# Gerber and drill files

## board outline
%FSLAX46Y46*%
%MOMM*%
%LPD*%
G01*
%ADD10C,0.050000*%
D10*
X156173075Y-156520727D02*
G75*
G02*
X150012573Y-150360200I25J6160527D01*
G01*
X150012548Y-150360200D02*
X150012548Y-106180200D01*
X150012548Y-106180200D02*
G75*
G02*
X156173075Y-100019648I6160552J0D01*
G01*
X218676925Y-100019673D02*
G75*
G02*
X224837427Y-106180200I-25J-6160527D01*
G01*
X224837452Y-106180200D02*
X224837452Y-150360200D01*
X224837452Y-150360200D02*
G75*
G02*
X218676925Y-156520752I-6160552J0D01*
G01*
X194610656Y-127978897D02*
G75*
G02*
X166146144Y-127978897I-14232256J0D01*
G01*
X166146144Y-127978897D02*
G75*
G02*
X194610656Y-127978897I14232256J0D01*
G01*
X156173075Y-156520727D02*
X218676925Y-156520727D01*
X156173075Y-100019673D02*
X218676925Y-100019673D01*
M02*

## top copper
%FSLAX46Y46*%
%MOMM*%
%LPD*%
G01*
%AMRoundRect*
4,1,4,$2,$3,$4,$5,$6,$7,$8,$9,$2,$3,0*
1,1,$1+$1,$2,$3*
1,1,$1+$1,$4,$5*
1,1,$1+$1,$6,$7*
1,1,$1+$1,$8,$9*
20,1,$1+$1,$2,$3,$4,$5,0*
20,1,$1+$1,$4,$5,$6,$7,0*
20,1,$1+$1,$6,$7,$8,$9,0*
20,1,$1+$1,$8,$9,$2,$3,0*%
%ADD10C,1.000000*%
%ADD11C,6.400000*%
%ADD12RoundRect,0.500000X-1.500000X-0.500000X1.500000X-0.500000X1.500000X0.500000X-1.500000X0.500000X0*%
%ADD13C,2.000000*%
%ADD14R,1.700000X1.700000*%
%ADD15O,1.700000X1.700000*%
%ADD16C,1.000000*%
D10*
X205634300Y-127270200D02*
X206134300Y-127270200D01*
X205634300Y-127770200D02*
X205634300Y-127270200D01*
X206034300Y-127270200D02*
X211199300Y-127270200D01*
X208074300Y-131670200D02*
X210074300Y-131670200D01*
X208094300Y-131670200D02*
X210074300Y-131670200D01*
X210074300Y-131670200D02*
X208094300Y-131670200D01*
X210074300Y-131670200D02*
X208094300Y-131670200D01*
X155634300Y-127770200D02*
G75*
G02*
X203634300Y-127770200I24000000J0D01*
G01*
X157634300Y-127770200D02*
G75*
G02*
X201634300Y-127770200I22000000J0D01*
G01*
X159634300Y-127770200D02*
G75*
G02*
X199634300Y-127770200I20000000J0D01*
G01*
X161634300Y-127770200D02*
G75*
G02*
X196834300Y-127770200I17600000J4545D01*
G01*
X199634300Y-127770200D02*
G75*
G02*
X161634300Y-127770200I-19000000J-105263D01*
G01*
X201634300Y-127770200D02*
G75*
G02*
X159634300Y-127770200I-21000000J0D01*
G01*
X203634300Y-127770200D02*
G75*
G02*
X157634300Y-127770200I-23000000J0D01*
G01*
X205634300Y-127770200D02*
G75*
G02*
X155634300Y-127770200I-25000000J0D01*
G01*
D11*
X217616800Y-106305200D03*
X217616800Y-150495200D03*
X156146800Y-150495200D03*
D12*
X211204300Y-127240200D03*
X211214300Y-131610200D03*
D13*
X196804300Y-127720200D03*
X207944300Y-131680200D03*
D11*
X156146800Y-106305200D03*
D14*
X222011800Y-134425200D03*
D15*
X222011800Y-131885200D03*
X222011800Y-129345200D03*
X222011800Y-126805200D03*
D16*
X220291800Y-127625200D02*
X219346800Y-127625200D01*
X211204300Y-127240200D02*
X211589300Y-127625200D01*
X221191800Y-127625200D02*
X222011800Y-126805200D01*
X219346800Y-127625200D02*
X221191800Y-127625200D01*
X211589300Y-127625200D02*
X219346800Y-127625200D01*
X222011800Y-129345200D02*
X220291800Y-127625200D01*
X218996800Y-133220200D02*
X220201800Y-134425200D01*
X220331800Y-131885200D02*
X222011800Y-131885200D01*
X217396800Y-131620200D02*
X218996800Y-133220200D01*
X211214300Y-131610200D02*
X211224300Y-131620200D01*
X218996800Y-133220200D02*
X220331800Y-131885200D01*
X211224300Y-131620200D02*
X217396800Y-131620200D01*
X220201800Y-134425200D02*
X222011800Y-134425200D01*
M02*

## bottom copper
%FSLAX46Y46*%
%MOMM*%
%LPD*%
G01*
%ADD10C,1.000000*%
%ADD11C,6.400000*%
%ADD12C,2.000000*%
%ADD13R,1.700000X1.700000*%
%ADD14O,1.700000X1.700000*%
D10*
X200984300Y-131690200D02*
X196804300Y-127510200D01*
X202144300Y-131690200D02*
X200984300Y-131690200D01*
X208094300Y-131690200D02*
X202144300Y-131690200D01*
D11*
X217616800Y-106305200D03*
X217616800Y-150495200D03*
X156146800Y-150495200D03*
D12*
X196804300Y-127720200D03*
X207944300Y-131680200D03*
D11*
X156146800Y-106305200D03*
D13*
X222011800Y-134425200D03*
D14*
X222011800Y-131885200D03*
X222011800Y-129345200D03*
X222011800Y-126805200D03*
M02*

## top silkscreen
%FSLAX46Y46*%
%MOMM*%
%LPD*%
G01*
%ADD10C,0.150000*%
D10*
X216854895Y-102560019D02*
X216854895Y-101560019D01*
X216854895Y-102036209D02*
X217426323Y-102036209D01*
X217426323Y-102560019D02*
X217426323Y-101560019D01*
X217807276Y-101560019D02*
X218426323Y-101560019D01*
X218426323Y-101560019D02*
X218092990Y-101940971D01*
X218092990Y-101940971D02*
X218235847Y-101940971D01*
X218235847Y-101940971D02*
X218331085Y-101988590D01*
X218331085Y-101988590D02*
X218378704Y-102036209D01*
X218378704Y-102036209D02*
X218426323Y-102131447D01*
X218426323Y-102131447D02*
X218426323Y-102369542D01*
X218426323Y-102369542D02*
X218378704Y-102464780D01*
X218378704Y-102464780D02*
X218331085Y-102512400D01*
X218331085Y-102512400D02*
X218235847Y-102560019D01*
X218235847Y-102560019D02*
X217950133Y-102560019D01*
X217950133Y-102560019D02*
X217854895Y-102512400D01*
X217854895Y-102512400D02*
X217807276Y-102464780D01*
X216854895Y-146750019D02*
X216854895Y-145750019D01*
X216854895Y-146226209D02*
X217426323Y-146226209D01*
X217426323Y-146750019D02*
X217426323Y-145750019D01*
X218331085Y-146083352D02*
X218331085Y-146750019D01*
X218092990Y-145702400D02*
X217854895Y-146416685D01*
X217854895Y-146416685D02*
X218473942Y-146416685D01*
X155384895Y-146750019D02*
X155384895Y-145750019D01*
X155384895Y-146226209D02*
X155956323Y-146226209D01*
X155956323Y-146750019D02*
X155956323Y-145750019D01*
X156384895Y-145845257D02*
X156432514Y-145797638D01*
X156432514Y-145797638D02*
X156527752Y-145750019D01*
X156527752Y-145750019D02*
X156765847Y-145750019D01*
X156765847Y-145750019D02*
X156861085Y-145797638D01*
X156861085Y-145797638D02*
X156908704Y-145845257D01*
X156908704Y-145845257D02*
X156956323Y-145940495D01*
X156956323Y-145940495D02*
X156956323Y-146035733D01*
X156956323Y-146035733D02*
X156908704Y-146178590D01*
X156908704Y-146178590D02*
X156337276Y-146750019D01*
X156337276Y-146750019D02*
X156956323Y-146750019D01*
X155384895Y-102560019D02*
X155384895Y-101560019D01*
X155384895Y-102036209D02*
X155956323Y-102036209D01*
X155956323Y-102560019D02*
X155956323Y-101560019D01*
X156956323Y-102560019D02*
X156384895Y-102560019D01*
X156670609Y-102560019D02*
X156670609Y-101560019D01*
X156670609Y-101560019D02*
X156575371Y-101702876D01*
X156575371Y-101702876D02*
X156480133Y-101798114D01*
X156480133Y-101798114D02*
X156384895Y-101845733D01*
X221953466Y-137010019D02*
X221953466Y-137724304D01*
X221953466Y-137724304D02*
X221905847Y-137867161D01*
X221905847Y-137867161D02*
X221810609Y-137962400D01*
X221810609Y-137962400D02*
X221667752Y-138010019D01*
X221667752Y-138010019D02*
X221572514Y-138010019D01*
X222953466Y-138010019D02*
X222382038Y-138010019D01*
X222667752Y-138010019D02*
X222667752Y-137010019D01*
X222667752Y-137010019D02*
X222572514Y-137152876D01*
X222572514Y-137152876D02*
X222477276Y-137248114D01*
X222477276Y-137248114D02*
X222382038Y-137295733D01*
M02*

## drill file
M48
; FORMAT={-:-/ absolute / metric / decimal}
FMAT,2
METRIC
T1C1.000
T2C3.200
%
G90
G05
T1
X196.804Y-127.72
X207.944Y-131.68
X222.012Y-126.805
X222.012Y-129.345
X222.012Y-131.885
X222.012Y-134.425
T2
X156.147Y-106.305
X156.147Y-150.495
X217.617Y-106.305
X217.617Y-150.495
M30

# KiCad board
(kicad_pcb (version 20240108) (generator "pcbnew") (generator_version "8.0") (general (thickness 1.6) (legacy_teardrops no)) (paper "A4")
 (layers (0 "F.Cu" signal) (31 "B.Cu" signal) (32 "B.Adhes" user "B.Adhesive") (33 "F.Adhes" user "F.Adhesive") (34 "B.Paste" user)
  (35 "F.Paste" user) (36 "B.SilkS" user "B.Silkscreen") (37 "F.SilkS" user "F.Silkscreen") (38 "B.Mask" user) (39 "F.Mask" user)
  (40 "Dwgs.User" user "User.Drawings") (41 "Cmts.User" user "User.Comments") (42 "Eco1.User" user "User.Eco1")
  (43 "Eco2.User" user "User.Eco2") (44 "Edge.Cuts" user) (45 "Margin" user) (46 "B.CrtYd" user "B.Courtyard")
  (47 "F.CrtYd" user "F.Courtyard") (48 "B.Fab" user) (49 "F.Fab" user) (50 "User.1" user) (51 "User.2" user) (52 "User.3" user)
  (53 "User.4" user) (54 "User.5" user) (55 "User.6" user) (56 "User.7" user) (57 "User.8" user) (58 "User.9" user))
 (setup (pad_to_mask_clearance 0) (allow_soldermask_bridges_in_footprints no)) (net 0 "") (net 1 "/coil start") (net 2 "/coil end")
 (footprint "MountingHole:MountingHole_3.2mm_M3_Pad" (layer "F.Cu") (at 217.6168 106.3052)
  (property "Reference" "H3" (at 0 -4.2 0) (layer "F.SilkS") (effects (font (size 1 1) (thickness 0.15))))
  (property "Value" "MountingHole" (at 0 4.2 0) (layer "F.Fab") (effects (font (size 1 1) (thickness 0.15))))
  (pad "1" thru_hole circle (at 0 0) (size 6.4 6.4) (drill 3.2) (layers "*.Cu" "*.Mask") (remove_unused_layers no)))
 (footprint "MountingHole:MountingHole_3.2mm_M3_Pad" (layer "F.Cu") (at 217.6168 150.4952)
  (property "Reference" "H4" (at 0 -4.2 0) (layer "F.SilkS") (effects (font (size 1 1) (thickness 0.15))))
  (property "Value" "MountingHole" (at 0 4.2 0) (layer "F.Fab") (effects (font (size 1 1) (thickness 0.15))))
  (pad "1" thru_hole circle (at 0 0) (size 6.4 6.4) (drill 3.2) (layers "*.Cu" "*.Mask") (remove_unused_layers no)))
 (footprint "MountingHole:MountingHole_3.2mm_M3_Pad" (layer "F.Cu") (at 156.1468 150.4952)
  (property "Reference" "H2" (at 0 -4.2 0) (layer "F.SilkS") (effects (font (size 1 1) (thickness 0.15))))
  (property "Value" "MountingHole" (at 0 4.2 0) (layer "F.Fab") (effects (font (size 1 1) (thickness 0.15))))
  (pad "1" thru_hole circle (at 0 0) (size 6.4 6.4) (drill 3.2) (layers "*.Cu" "*.Mask") (remove_unused_layers no)))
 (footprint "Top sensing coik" (layer "F.Cu") (at 179.6343 127.7702)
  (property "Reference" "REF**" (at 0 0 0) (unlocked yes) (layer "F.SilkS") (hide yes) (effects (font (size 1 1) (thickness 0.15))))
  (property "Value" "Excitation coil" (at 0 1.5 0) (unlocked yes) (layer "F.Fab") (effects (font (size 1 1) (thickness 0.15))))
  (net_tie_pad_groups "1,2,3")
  (fp_line (start 26 -0.5) (end 26.5 -0.5) (stroke (width 1) (type solid)) (layer "F.Cu"))
  (fp_line (start 26 0) (end 26 -0.5) (stroke (width 1) (type solid)) (layer "F.Cu"))
  (fp_line (start 26.4 -0.5) (end 31.565 -0.5) (stroke (width 1) (type default)) (layer "F.Cu"))
  (fp_line (start 28.44 3.9) (end 30.44 3.9) (stroke (width 1) (type default)) (layer "F.Cu"))
  (fp_line (start 28.46 3.9) (end 30.44 3.9) (stroke (width 1) (type default)) (layer "F.Cu"))
  (fp_line (start 30.44 3.9) (end 28.46 3.9) (stroke (width 1) (type default)) (layer "F.Cu"))
  (fp_line (start 30.44 3.9) (end 28.46 3.9) (stroke (width 1) (type default)) (layer "F.Cu"))
  (fp_arc (start -24 0) (mid 0 -24) (end 24 0) (stroke (width 1) (type solid)) (layer "F.Cu"))
  (fp_arc (start -22 0) (mid 0 -22) (end 22 0) (stroke (width 1) (type solid)) (layer "F.Cu"))
  (fp_arc (start -20 0) (mid 0 -20) (end 20 0) (stroke (width 1) (type solid)) (layer "F.Cu"))
  (fp_arc (start -18 0) (mid -0.4 -17.604546) (end 17.2 0) (stroke (width 1) (type solid)) (layer "F.Cu"))
  (fp_arc (start 20 0) (mid 1 19.105555) (end -18 0) (stroke (width 1) (type solid)) (layer "F.Cu"))
  (fp_arc (start 22 0) (mid 1 21) (end -20 0) (stroke (width 1) (type solid)) (layer "F.Cu"))
  (fp_arc (start 24 0) (mid 1 23) (end -22 0) (stroke (width 1) (type solid)) (layer "F.Cu"))
  (fp_arc (start 26 0) (mid 1 25) (end -24 0) (stroke (width 1) (type solid)) (layer "F.Cu"))
  (fp_line (start 21.35 3.92) (end 17.17 -0.26) (stroke (width 1) (type default)) (layer "B.Cu"))
  (fp_line (start 22.51 3.92) (end 21.35 3.92) (stroke (width 1) (type default)) (layer "B.Cu"))
  (fp_line (start 28.46 3.92) (end 22.51 3.92) (stroke (width 1) (type default)) (layer "B.Cu"))
  (pad "1" smd roundrect (at 31.57 -0.53) (size 4 2) (layers "F.Cu") (roundrect_rratio 0.25) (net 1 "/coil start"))
  (pad "2" smd roundrect (at 31.58 3.84) (size 4 2) (layers "F.Cu") (roundrect_rratio 0.25) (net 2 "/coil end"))
  (pad "3" thru_hole circle (at 17.17 -0.05 90) (size 2 2) (drill 1) (layers "*.Cu" "*.Mask") (remove_unused_layers no))
  (pad "3" thru_hole circle (at 28.31 3.91 90) (size 2 2) (drill 1) (layers "*.Cu" "*.Mask") (remove_unused_layers no)))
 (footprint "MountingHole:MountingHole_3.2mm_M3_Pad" (layer "F.Cu") (at 156.1468 106.3052)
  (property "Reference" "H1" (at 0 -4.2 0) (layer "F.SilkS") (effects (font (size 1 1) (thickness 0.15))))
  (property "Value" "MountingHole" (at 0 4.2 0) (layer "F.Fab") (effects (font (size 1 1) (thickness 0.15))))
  (pad "1" thru_hole circle (at 0 0) (size 6.4 6.4) (drill 3.2) (layers "*.Cu" "*.Mask") (remove_unused_layers no)))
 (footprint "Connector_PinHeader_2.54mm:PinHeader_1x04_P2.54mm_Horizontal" (layer "B.Cu") (at 222.0118 134.4252)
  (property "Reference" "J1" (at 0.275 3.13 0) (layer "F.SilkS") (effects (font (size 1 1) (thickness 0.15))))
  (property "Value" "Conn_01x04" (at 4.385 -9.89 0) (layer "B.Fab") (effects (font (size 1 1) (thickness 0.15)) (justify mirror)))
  (pad "1" thru_hole rect (at 0 0) (size 1.7 1.7) (drill 1) (layers "*.Cu" "*.Mask") (remove_unused_layers no) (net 2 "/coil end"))
  (pad "2" thru_hole oval (at 0 -2.54) (size 1.7 1.7) (drill 1) (layers "*.Cu" "*.Mask") (remove_unused_layers no) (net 2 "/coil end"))
  (pad "3" thru_hole oval (at 0 -5.08) (size 1.7 1.7) (drill 1) (layers "*.Cu" "*.Mask") (remove_unused_layers no) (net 1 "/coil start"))
  (pad "4" thru_hole oval (at 0 -7.62) (size 1.7 1.7) (drill 1) (layers "*.Cu" "*.Mask") (remove_unused_layers no) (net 1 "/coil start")))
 (gr_arc (start 156.173075 156.520727) (mid 151.816925 154.71635) (end 150.012548 150.3602) (stroke (width 0.05) (type default))
  (layer "Edge.Cuts"))
 (gr_line (start 150.012548 150.3602) (end 150.012548 106.1802) (stroke (width 0.05) (type default)) (layer "Edge.Cuts"))
 (gr_arc (start 150.012548 106.1802) (mid 151.816925 101.82405) (end 156.173075 100.019673) (stroke (width 0.05) (type default))
  (layer "Edge.Cuts"))
 (gr_arc (start 218.676925 100.019673) (mid 223.033075 101.82405) (end 224.837452 106.1802) (stroke (width 0.05) (type default))
  (layer "Edge.Cuts"))
 (gr_line (start 224.837452 106.1802) (end 224.837452 150.3602) (stroke (width 0.05) (type default)) (layer "Edge.Cuts"))
 (gr_arc (start 224.837452 150.3602) (mid 223.033075 154.71635) (end 218.676925 156.520727) (stroke (width 0.05) (type default))
  (layer "Edge.Cuts"))
 (gr_circle (center 180.3784 127.978897) (end 192.7568 120.9552) (stroke (width 0.05) (type default)) (fill none) (layer "Edge.Cuts"))
 (gr_line (start 156.173075 156.520727) (end 218.676925 156.520727) (stroke (width 0.05) (type default)) (layer "Edge.Cuts"))
 (gr_line (start 156.173075 100.019673) (end 218.676925 100.019673) (stroke (width 0.05) (type default)) (layer "Edge.Cuts"))
 (segment (start 220.2918 127.6252) (end 219.3468 127.6252) (width 1) (layer "F.Cu") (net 1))
 (segment (start 211.2043 127.2402) (end 211.5893 127.6252) (width 1) (layer "F.Cu") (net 1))
 (segment (start 221.1918 127.6252) (end 222.0118 126.8052) (width 1) (layer "F.Cu") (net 1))
 (segment (start 219.3468 127.6252) (end 221.1918 127.6252) (width 1) (layer "F.Cu") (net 1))
 (segment (start 211.5893 127.6252) (end 219.3468 127.6252) (width 1) (layer "F.Cu") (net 1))
 (segment (start 222.0118 129.3452) (end 220.2918 127.6252) (width 1) (layer "F.Cu") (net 1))
 (segment (start 218.9968 133.2202) (end 220.2018 134.4252) (width 1) (layer "F.Cu") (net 2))
 (segment (start 220.3318 131.8852) (end 222.0118 131.8852) (width 1) (layer "F.Cu") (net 2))
 (segment (start 217.3968 131.6202) (end 218.9968 133.2202) (width 1) (layer "F.Cu") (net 2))
 (segment (start 211.2143 131.6102) (end 211.2243 131.6202) (width 1) (layer "F.Cu") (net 2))
 (segment (start 218.9968 133.2202) (end 220.3318 131.8852) (width 1) (layer "F.Cu") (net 2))
 (segment (start 211.2243 131.6202) (end 217.3968 131.6202) (width 1) (layer "F.Cu") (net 2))
 (segment (start 220.2018 134.4252) (end 222.0118 134.4252) (width 1) (layer "F.Cu") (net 2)))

